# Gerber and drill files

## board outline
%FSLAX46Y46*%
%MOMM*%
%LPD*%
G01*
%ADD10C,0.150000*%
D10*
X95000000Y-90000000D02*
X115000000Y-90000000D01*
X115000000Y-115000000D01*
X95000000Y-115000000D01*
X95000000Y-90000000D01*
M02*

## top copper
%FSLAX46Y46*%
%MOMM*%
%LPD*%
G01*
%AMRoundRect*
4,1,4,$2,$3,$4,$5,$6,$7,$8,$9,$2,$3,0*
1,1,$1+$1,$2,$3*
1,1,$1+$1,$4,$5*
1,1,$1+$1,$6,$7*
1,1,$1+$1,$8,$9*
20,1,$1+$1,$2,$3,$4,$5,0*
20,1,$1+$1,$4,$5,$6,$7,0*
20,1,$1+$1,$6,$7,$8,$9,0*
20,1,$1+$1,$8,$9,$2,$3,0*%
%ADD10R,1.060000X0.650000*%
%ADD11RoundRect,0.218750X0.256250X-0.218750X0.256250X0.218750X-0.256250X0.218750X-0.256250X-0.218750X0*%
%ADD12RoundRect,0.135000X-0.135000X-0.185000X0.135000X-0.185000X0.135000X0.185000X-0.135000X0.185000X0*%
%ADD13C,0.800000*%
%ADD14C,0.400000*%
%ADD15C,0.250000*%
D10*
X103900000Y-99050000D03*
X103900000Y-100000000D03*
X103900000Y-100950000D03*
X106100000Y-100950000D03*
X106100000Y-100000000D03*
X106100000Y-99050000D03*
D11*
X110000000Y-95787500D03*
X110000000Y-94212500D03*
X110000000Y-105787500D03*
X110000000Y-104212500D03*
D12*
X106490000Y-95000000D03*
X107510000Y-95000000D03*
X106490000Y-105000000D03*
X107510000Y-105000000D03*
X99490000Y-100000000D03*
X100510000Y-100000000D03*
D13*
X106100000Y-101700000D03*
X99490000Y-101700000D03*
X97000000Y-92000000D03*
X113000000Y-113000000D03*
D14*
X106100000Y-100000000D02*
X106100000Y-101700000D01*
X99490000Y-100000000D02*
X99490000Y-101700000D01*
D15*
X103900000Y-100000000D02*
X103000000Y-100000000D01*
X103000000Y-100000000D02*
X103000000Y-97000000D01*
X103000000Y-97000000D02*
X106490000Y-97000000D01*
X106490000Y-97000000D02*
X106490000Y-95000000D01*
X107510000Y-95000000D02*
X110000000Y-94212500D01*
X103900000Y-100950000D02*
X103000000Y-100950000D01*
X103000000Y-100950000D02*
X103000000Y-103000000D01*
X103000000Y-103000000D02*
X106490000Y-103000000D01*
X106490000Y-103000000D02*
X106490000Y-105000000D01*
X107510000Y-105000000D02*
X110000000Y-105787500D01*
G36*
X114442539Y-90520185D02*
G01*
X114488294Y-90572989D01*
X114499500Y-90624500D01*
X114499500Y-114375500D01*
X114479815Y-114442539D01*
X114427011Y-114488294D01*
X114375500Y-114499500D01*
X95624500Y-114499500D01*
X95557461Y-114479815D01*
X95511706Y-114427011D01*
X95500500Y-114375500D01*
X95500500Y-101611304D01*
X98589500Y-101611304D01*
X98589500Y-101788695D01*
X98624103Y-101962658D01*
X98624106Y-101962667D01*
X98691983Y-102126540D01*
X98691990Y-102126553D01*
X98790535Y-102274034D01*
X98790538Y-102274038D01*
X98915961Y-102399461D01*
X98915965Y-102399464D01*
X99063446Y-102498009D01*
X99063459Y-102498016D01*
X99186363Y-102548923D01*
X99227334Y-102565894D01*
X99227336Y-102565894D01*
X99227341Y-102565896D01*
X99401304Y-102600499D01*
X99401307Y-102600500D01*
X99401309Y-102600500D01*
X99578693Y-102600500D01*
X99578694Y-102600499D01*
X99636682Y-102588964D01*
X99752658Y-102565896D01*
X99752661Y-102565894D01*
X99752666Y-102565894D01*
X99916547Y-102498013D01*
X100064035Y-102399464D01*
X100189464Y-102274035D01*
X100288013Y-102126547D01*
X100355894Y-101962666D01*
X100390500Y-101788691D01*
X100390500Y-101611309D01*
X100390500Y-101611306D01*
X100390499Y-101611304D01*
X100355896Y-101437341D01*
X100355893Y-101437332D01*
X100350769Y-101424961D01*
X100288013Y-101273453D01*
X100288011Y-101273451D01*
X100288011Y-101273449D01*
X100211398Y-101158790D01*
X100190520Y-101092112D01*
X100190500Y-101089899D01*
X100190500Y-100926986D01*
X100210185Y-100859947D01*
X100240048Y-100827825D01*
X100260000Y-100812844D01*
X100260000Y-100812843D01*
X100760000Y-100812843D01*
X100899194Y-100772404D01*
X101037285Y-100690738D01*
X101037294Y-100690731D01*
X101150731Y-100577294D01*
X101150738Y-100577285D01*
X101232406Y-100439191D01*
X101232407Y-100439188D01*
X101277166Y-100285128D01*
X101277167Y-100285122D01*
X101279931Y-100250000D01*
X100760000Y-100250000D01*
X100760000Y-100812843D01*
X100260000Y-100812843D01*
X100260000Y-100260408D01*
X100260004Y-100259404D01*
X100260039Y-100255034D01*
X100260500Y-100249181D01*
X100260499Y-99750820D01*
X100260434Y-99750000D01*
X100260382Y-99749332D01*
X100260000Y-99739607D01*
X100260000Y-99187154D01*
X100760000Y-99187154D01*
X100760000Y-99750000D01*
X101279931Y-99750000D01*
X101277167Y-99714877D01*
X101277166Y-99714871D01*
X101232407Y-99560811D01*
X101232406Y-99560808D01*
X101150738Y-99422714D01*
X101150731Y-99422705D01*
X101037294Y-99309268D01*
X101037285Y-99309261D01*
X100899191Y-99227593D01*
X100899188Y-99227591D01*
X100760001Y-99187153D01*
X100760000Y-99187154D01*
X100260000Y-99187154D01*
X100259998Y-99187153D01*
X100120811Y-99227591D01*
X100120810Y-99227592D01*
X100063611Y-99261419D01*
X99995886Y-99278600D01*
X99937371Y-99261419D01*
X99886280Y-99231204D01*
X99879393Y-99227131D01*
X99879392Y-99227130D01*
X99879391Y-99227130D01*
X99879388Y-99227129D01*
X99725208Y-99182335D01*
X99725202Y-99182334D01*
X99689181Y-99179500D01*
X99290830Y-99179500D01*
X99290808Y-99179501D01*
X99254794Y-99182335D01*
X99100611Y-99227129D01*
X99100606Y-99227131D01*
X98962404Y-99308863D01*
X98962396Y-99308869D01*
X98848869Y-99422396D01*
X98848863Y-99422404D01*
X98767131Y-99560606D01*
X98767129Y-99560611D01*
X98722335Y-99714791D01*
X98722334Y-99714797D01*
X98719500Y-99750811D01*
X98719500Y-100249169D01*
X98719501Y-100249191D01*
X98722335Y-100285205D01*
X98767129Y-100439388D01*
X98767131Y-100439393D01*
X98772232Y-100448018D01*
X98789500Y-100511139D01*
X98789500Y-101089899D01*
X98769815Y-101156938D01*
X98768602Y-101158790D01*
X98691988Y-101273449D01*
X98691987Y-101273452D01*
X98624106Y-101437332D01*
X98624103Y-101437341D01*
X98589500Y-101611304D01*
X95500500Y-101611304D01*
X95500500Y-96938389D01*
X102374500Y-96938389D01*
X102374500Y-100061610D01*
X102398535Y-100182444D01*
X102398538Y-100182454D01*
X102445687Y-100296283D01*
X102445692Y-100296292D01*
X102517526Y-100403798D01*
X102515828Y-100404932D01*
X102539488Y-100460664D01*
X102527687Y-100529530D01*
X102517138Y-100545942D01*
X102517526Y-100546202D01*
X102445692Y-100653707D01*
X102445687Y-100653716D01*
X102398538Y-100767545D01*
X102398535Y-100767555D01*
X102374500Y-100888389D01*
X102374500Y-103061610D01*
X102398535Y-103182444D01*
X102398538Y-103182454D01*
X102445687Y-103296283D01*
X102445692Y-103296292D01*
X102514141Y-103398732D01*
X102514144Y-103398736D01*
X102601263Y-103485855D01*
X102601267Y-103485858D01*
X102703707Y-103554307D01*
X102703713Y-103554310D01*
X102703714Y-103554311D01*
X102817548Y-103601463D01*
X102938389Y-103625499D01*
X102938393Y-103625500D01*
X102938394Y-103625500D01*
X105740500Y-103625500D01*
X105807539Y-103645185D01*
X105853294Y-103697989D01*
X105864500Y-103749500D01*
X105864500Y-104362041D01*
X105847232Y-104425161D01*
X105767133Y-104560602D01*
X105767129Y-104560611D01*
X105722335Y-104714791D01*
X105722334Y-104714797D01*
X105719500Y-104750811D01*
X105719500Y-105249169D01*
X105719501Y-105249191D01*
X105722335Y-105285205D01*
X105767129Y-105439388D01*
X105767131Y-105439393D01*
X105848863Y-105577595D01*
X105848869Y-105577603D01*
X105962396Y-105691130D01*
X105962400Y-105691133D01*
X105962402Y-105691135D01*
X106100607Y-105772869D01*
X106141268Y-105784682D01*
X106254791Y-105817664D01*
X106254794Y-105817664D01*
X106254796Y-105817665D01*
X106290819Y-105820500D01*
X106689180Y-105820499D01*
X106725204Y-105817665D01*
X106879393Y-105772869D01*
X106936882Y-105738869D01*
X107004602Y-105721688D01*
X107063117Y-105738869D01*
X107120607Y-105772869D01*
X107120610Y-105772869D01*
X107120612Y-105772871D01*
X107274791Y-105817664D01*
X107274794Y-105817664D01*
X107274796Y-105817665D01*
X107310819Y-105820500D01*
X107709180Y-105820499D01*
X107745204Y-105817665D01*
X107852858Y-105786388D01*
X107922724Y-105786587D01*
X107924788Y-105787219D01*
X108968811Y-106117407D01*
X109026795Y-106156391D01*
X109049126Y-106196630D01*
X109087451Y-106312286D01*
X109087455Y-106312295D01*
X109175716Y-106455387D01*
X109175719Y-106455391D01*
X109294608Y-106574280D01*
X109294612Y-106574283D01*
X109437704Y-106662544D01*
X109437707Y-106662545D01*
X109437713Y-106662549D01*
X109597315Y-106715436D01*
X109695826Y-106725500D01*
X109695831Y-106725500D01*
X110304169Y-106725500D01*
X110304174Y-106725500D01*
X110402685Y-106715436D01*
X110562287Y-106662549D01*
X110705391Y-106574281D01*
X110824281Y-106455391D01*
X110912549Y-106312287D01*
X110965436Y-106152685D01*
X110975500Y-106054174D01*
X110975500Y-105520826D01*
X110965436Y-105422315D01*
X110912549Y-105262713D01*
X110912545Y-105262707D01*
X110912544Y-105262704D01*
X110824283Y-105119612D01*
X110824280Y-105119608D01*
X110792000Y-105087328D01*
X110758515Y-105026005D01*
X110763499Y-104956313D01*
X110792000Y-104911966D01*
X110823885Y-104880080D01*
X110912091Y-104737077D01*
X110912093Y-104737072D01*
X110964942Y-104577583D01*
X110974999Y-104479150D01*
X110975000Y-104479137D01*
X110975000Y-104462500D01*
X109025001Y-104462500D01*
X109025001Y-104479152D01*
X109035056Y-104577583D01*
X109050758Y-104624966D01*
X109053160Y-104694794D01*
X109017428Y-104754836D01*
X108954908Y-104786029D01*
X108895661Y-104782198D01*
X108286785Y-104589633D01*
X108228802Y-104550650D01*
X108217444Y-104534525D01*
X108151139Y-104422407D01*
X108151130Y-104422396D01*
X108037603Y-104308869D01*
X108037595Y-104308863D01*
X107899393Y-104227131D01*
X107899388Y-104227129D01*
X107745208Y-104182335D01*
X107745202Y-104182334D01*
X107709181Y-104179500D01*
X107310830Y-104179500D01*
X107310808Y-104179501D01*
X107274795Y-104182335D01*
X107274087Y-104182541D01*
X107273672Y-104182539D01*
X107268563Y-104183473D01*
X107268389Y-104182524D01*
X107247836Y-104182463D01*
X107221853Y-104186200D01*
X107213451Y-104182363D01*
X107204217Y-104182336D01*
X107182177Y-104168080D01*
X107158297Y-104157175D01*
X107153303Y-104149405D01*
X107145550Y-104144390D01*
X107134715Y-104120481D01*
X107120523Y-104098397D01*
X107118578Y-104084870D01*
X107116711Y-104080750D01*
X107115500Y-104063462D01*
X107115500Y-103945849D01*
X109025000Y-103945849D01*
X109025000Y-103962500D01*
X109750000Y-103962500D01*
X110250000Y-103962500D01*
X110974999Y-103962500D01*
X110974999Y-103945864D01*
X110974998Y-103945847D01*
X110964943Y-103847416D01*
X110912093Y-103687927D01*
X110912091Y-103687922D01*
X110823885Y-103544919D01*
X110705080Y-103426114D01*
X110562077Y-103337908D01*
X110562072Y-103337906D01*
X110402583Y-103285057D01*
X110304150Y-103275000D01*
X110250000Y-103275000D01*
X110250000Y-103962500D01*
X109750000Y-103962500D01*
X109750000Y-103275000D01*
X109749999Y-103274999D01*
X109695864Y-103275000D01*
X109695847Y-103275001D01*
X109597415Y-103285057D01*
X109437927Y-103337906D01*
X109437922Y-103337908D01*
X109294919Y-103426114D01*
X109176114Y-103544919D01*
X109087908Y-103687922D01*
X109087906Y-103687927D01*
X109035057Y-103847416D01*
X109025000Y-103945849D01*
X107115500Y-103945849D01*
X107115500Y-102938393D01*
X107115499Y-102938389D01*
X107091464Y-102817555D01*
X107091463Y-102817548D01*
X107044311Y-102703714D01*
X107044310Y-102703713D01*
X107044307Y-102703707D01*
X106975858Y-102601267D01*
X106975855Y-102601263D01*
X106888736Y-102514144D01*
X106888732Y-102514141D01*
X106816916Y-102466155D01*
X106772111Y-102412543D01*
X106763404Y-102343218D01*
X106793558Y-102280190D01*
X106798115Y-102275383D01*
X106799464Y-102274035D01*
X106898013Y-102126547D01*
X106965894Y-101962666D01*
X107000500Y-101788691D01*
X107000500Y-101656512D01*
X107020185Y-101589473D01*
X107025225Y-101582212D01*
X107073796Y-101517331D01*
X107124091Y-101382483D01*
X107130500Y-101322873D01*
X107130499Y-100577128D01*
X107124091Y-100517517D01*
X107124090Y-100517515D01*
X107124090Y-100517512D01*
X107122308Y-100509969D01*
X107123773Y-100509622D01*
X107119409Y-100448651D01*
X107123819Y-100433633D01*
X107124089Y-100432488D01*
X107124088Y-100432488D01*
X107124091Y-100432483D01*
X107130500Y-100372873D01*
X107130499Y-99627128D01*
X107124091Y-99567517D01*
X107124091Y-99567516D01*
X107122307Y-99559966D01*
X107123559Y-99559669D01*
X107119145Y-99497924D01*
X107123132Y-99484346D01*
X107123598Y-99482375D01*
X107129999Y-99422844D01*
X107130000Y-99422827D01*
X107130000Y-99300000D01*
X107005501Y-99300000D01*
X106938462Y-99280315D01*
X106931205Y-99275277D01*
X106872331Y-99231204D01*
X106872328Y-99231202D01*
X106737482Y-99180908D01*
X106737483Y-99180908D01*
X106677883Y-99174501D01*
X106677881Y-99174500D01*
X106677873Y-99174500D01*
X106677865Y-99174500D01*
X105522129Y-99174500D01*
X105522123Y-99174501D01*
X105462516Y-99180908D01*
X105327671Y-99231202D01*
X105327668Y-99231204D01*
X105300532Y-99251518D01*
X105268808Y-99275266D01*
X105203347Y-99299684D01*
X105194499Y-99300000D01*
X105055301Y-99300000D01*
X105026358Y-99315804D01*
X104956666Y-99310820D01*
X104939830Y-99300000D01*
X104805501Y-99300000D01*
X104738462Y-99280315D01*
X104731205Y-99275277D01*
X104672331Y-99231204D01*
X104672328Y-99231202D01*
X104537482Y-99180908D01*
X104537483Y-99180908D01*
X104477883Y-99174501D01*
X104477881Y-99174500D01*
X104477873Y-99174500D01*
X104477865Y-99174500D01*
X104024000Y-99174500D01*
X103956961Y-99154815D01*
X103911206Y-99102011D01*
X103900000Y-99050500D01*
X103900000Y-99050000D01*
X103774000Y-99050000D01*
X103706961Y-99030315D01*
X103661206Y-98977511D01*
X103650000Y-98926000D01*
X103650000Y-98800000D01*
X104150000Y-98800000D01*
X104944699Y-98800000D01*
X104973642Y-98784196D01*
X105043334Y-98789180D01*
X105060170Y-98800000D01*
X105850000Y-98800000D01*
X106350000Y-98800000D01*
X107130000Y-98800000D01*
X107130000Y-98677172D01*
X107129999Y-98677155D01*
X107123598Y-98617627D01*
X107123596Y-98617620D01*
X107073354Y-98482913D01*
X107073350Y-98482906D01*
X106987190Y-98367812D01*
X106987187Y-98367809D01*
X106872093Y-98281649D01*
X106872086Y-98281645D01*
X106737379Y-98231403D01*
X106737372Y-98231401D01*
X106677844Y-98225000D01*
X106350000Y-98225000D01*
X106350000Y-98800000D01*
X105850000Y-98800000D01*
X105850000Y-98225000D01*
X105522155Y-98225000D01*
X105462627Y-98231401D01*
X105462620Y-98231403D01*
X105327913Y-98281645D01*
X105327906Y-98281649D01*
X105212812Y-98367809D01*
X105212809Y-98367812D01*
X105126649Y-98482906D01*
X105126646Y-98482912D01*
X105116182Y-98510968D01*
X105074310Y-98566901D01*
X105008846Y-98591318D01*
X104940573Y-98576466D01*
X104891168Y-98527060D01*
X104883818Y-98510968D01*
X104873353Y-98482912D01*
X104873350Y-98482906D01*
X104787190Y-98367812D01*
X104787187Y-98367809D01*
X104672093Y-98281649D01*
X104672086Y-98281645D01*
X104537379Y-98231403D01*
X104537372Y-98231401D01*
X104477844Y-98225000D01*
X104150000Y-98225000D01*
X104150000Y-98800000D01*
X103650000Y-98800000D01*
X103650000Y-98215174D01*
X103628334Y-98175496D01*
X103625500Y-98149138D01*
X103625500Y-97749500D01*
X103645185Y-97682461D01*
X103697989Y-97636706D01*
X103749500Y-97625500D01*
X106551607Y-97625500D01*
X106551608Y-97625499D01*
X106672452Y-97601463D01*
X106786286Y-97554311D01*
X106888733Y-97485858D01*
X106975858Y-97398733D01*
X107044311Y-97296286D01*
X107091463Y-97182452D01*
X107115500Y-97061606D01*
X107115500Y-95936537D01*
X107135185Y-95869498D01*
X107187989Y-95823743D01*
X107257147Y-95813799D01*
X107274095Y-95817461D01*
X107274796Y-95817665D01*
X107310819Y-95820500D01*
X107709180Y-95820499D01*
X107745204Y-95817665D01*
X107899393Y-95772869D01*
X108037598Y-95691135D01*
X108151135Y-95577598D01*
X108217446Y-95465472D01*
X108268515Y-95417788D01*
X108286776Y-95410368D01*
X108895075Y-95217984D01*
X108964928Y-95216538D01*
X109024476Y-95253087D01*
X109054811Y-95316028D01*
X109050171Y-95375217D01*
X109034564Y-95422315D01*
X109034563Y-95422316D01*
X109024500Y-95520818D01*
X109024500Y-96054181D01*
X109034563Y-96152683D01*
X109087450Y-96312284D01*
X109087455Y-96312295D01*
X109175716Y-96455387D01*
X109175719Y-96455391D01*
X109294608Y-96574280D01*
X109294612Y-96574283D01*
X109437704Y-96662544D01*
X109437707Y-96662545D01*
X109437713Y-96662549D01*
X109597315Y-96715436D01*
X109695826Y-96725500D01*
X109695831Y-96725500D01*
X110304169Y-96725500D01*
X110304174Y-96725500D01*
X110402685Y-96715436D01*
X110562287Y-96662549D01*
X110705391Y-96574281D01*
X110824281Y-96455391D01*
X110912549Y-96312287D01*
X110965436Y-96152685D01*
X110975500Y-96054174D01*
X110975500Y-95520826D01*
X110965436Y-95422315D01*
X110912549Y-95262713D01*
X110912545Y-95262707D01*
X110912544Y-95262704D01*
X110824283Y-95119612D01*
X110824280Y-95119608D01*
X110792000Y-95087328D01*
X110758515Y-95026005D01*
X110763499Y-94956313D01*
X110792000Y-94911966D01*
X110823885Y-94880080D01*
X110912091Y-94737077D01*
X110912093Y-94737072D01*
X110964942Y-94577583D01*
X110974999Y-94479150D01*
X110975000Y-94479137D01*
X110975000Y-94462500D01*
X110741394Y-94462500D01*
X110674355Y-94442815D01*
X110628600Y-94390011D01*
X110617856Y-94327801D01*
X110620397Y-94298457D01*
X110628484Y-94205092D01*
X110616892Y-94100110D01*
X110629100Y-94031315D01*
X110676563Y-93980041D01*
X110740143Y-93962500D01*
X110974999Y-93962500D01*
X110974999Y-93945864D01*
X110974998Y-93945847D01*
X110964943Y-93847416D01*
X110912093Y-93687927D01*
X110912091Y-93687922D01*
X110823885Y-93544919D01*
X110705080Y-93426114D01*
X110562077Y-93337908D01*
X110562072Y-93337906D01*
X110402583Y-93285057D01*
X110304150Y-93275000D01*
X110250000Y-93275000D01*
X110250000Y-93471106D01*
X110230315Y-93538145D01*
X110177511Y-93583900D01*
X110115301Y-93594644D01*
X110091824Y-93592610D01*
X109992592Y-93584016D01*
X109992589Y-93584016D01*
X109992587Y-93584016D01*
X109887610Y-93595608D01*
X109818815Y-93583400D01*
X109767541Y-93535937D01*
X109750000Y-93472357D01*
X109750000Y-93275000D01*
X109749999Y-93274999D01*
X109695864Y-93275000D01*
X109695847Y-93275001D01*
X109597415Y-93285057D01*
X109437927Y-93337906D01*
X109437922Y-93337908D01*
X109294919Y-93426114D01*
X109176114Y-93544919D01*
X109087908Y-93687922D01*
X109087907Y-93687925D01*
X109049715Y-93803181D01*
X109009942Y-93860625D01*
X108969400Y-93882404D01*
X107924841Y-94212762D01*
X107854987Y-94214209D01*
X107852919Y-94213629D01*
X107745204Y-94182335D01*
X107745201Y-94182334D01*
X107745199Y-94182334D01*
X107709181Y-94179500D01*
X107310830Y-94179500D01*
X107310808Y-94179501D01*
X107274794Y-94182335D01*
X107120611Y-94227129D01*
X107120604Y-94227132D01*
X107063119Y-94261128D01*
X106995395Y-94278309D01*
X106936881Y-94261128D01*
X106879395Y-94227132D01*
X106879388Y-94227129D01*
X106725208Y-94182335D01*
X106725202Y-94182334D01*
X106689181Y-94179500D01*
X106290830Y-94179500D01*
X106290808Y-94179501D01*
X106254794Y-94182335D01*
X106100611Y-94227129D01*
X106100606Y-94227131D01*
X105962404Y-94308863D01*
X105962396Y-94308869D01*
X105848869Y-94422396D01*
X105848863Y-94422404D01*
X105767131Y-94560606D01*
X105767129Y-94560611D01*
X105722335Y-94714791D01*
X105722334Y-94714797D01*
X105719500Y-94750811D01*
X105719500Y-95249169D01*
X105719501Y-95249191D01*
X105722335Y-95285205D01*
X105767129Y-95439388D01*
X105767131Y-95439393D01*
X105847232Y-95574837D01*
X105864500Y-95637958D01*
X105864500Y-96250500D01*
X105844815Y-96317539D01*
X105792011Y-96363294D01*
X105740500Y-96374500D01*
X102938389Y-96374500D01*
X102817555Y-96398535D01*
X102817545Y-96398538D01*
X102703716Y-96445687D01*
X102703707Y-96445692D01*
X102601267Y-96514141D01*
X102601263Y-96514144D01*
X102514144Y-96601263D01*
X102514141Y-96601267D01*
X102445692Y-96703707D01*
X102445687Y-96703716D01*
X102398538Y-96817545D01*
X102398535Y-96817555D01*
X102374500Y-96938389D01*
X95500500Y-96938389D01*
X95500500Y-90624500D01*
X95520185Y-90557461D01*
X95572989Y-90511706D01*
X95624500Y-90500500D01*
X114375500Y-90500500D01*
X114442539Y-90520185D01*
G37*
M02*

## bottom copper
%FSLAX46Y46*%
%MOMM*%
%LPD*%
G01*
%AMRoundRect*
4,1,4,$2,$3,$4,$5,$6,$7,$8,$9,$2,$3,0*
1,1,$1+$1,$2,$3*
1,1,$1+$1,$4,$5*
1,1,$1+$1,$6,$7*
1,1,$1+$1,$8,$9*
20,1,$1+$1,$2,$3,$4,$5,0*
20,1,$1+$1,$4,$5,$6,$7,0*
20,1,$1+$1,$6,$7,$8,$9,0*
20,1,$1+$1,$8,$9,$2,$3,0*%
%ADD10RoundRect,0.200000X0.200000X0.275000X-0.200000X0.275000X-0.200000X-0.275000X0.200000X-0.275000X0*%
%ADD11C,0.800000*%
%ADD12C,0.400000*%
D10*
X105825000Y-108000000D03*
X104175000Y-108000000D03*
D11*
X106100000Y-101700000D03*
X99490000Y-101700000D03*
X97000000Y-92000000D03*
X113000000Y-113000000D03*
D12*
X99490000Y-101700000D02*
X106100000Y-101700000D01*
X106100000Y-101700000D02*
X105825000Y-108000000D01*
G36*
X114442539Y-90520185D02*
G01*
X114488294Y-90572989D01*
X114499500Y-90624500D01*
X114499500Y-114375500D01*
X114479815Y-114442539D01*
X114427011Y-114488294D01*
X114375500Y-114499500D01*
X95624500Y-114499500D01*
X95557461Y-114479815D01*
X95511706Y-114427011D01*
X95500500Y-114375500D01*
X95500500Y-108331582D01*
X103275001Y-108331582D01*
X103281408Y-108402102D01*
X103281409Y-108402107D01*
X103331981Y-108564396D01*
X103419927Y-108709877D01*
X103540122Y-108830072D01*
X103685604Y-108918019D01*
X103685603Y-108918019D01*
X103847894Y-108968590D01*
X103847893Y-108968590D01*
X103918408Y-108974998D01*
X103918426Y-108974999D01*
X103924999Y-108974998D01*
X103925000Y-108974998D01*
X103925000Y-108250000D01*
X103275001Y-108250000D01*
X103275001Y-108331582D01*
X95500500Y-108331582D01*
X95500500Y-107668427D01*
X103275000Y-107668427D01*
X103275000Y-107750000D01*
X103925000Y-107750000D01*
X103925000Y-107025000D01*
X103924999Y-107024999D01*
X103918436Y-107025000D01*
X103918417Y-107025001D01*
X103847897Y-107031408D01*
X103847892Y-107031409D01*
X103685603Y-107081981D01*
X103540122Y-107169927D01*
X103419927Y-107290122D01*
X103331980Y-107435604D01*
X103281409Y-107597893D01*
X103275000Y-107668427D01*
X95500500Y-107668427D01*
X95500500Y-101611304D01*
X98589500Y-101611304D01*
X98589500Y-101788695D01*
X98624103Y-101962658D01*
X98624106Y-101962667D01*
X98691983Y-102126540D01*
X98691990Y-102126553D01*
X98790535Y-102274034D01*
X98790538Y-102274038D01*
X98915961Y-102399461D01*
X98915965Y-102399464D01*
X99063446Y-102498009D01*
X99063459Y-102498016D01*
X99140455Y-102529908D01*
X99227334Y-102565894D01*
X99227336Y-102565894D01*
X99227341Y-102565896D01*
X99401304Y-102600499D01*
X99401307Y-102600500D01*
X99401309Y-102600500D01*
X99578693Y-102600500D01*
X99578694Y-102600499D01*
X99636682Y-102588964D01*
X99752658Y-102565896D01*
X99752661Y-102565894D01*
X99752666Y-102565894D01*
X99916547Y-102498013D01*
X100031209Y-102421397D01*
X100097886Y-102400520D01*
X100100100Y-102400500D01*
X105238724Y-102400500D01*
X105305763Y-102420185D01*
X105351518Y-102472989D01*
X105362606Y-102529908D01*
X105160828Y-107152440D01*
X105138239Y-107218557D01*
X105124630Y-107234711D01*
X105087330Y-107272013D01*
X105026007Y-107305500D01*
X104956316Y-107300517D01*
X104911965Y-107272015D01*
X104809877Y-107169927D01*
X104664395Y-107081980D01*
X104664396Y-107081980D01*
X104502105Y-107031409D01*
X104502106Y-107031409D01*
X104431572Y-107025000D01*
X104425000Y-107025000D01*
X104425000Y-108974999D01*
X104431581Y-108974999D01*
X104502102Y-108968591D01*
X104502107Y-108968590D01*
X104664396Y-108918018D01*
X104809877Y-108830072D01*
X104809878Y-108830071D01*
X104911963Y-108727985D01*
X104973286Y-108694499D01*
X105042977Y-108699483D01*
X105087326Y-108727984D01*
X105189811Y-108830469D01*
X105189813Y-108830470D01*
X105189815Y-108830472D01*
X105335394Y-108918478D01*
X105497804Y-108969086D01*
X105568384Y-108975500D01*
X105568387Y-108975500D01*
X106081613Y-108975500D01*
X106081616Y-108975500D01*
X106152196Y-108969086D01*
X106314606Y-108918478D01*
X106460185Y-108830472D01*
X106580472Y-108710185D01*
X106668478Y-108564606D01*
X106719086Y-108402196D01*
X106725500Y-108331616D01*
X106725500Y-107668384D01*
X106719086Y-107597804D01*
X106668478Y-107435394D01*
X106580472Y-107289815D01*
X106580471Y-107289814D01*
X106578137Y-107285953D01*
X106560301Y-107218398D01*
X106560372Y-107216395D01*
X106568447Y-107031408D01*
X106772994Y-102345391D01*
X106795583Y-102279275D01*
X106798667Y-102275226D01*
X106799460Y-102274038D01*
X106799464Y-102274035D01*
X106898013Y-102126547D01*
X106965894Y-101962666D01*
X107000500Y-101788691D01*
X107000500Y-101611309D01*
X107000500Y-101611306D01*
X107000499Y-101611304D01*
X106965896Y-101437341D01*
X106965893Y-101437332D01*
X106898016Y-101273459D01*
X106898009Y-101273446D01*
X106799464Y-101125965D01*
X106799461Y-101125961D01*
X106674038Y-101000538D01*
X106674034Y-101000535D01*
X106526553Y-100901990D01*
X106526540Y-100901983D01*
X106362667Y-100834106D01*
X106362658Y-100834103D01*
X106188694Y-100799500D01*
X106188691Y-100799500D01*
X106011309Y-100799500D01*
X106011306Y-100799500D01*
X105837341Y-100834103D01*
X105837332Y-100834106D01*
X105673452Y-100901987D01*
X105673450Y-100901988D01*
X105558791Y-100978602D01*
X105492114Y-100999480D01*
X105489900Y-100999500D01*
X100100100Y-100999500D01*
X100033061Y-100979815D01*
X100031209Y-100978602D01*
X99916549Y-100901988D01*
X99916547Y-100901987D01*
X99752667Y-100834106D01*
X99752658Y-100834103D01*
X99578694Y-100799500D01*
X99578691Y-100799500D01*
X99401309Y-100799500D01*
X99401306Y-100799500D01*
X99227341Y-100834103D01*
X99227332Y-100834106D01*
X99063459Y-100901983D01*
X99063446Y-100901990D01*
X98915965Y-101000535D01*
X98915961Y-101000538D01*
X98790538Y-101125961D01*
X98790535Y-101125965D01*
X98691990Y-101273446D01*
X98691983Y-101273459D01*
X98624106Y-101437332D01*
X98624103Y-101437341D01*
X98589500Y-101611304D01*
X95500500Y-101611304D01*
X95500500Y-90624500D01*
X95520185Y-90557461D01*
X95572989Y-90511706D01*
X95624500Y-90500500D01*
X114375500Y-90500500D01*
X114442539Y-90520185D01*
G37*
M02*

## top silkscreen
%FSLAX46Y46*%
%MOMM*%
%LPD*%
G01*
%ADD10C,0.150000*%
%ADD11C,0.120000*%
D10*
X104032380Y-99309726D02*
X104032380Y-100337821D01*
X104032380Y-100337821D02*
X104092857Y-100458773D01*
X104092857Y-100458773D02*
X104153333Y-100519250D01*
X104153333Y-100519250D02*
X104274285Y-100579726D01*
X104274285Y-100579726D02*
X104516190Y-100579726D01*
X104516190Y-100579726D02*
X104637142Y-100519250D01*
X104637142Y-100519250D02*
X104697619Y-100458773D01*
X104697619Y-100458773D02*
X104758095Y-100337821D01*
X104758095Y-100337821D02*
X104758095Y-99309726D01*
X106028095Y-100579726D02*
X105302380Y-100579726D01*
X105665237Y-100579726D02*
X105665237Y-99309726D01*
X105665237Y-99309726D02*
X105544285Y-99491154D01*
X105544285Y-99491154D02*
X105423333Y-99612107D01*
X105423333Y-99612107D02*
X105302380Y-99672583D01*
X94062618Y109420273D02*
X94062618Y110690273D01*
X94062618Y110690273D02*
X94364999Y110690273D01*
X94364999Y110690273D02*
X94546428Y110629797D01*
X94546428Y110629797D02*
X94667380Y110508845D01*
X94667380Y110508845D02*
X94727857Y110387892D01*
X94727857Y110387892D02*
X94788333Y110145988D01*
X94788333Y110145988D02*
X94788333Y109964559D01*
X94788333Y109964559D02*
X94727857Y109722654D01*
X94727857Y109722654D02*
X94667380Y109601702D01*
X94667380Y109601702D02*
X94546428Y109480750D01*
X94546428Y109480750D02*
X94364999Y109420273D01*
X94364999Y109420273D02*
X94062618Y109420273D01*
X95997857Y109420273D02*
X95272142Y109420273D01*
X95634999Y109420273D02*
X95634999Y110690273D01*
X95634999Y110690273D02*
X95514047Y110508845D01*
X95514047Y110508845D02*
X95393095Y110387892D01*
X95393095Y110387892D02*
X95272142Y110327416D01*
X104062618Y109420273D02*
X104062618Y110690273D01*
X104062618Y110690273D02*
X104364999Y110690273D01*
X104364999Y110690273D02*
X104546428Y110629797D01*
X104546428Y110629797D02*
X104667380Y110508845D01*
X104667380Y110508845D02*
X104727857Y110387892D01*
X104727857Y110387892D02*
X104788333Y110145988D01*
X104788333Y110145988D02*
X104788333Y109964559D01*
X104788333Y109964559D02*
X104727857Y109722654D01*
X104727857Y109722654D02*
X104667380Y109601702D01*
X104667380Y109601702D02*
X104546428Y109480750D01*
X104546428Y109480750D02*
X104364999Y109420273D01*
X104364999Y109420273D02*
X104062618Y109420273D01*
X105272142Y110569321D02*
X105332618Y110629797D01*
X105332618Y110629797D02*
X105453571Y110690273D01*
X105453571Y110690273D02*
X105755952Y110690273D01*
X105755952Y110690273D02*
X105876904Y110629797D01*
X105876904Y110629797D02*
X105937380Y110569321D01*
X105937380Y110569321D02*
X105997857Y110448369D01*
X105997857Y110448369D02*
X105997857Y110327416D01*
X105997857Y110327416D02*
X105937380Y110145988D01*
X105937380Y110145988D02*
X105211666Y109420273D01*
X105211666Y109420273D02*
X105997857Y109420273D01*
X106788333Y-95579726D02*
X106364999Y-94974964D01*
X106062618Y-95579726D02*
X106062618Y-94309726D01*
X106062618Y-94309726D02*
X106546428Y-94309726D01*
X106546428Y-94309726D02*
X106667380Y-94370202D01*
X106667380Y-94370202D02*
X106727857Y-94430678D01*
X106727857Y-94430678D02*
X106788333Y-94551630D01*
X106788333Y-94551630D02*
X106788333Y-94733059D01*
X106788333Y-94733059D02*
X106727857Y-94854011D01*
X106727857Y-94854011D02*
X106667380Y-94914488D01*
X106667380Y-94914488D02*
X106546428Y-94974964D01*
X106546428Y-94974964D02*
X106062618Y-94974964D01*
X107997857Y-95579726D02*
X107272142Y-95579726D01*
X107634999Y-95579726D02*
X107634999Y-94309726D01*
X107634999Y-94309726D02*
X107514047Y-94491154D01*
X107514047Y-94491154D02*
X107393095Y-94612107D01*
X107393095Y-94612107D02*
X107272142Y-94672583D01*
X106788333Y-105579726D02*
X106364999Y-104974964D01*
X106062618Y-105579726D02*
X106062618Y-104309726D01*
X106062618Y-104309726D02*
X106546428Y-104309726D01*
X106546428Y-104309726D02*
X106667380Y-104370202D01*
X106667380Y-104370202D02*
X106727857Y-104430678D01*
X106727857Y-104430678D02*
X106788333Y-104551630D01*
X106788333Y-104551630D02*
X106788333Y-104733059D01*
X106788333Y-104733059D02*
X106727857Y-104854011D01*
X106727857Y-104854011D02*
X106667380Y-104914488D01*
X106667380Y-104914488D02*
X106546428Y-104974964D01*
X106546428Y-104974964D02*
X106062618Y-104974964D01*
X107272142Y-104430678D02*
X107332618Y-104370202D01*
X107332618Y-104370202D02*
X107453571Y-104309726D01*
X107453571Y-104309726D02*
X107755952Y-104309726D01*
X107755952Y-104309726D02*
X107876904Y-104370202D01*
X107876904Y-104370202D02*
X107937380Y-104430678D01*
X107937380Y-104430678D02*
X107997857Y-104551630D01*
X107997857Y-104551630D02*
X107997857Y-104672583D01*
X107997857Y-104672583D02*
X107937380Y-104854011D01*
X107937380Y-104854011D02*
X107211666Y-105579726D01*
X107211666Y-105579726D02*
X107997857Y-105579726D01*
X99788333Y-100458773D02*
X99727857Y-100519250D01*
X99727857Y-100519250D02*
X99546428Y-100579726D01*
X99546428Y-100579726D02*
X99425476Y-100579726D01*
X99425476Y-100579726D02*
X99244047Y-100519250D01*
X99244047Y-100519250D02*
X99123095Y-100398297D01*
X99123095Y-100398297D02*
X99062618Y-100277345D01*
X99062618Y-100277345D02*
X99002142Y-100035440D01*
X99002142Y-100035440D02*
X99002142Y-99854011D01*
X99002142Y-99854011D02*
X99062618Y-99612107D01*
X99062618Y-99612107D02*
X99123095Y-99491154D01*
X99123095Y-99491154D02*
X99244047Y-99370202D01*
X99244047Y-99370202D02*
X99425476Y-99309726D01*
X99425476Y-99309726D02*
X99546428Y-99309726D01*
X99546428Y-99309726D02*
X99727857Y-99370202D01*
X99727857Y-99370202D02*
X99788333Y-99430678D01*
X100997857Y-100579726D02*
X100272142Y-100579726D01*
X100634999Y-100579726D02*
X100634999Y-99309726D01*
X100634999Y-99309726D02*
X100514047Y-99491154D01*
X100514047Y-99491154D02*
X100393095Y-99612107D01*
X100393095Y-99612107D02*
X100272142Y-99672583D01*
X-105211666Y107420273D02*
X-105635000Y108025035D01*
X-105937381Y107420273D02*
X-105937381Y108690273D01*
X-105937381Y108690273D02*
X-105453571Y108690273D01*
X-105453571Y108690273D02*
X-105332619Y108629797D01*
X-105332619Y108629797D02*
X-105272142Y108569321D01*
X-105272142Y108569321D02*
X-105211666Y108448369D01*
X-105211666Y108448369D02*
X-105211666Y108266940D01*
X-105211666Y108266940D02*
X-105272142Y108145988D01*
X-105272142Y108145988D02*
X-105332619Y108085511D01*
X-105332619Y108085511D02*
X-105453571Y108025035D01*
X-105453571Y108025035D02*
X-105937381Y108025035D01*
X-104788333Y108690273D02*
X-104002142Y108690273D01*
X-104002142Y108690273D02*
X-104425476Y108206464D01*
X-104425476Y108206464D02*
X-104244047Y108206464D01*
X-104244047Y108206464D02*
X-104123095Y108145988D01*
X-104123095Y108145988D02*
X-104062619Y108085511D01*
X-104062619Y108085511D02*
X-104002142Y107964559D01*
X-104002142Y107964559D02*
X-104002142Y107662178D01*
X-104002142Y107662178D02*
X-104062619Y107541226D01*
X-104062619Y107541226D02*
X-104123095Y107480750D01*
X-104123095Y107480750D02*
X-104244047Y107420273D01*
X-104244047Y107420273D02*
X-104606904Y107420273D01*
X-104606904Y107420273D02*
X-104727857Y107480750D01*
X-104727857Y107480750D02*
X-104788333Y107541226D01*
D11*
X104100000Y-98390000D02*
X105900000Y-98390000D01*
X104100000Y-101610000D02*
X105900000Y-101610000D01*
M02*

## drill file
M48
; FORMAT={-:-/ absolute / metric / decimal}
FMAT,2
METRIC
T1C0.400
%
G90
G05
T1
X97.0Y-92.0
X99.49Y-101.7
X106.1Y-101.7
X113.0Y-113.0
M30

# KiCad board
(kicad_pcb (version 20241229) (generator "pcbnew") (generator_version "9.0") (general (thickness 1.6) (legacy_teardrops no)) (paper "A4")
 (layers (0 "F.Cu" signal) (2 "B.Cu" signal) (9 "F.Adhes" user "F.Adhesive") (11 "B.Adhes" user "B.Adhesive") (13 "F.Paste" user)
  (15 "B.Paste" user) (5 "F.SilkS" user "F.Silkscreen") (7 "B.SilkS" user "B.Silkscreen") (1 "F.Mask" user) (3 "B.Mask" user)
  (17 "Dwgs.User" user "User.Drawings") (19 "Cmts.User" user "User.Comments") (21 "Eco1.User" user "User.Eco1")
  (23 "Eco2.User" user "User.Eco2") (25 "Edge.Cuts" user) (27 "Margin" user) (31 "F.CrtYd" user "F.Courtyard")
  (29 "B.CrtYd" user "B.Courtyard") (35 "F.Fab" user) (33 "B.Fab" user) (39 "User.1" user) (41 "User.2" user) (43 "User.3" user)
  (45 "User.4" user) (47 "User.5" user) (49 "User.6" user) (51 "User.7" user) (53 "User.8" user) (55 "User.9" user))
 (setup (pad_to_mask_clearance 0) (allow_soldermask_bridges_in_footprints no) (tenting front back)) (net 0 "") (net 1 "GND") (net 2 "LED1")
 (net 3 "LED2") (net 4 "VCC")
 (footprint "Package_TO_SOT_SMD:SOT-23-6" (layer "F.Cu") (at 105 100)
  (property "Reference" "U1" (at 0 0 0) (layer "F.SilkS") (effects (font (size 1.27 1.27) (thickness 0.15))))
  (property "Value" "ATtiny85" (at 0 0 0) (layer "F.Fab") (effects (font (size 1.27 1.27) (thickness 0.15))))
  (fp_line (start -0.9 -1.61) (end 0.9 -1.61) (stroke (width 0.12) (type solid)) (layer "F.SilkS"))
  (fp_line (start -0.9 1.61) (end 0.9 1.61) (stroke (width 0.12) (type solid)) (layer "F.SilkS"))
  (pad "1" smd rect (at -1.1 -0.95) (size 1.06 0.65) (layers "F.Cu" "F.Mask" "F.Paste") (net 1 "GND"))
  (pad "2" smd rect (at -1.1 0) (size 1.06 0.65) (layers "F.Cu" "F.Mask" "F.Paste") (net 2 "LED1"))
  (pad "3" smd rect (at -1.1 0.95) (size 1.06 0.65) (layers "F.Cu" "F.Mask" "F.Paste") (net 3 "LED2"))
  (pad "4" smd rect (at 1.1 0.95) (size 1.06 0.65) (layers "F.Cu" "F.Mask" "F.Paste") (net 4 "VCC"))
  (pad "5" smd rect (at 1.1 0) (size 1.06 0.65) (layers "F.Cu" "F.Mask" "F.Paste") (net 4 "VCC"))
  (pad "6" smd rect (at 1.1 -0.95) (size 1.06 0.65) (layers "F.Cu" "F.Mask" "F.Paste") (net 1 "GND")))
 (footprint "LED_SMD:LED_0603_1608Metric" (layer "F.Cu") (at 110 95 90)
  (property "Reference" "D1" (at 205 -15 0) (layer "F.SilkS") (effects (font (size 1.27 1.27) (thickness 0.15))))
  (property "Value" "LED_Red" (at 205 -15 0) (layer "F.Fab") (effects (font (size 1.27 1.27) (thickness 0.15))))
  (pad "1" smd roundrect (at -0.7875 0 90) (size 0.875 0.95) (layers "F.Cu" "F.Mask" "F.Paste") (roundrect_rratio 0.25) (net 2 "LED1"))
  (pad "2" smd roundrect (at 0.7875 0 90) (size 0.875 0.95) (layers "F.Cu" "F.Mask" "F.Paste") (roundrect_rratio 0.25) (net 1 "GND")))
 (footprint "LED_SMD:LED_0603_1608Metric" (layer "F.Cu") (at 110 105 90)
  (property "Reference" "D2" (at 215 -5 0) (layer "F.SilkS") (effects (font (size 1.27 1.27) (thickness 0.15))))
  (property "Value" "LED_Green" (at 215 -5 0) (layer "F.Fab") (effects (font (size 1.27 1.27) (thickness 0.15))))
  (pad "1" smd roundrect (at -0.7875 0 90) (size 0.875 0.95) (layers "F.Cu" "F.Mask" "F.Paste") (roundrect_rratio 0.25) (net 3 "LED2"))
  (pad "2" smd roundrect (at 0.7875 0 90) (size 0.875 0.95) (layers "F.Cu" "F.Mask" "F.Paste") (roundrect_rratio 0.25) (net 1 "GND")))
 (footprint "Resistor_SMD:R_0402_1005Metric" (layer "F.Cu") (at 107 95)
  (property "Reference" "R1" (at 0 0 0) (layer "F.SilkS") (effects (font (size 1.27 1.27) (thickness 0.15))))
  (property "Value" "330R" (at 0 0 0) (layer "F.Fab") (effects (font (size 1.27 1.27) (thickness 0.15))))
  (pad "1" smd roundrect (at -0.51 0) (size 0.54 0.64) (layers "F.Cu" "F.Mask" "F.Paste") (roundrect_rratio 0.25) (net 2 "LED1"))
  (pad "2" smd roundrect (at 0.51 0) (size 0.54 0.64) (layers "F.Cu" "F.Mask" "F.Paste") (roundrect_rratio 0.25) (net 2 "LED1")))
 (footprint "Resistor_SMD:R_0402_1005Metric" (layer "F.Cu") (at 107 105)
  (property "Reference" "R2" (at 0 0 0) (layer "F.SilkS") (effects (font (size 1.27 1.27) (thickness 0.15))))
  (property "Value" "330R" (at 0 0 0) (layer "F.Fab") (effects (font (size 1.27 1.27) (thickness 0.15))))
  (pad "1" smd roundrect (at -0.51 0) (size 0.54 0.64) (layers "F.Cu" "F.Mask" "F.Paste") (roundrect_rratio 0.25) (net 3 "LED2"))
  (pad "2" smd roundrect (at 0.51 0) (size 0.54 0.64) (layers "F.Cu" "F.Mask" "F.Paste") (roundrect_rratio 0.25) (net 3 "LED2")))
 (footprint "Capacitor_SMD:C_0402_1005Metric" (layer "F.Cu") (at 100 100)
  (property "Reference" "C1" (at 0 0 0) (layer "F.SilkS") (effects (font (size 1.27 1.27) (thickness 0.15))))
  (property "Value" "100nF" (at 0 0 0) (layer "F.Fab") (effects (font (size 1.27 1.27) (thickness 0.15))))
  (pad "1" smd roundrect (at -0.51 0) (size 0.54 0.64) (layers "F.Cu" "F.Mask" "F.Paste") (roundrect_rratio 0.25) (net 4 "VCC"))
  (pad "2" smd roundrect (at 0.51 0) (size 0.54 0.64) (layers "F.Cu" "F.Mask" "F.Paste") (roundrect_rratio 0.25) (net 1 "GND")))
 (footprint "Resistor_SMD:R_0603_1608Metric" (layer "B.Cu") (at 105 108 180)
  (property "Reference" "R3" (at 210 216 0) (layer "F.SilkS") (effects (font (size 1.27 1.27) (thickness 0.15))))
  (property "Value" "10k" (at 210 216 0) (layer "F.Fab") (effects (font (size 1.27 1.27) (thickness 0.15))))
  (pad "1" smd roundrect (at -0.825 0 180) (size 0.8 0.95) (layers "B.Cu" "B.Mask" "B.Paste") (roundrect_rratio 0.25) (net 4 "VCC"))
  (pad "2" smd roundrect (at 0.825 0 180) (size 0.8 0.95) (layers "B.Cu" "B.Mask" "B.Paste") (roundrect_rratio 0.25) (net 1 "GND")))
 (gr_rect (start 95 90) (end 115 115) (stroke (width 0.15) (type solid)) (fill no) (layer "Edge.Cuts"))
 (segment (start 106.1 100) (end 106.1 101.7) (width 0.4) (layer "F.Cu") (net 4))
 (segment (start 99.49 100) (end 99.49 101.7) (width 0.4) (layer "F.Cu") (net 4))
 (via (at 106.1 101.7) (size 0.8) (drill 0.4) (layers "F.Cu" "B.Cu") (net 4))
 (via (at 99.49 101.7) (size 0.8) (drill 0.4) (layers "F.Cu" "B.Cu") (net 4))
 (segment (start 99.49 101.7) (end 106.1 101.7) (width 0.4) (layer "B.Cu") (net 4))
 (segment (start 106.1 101.7) (end 105.825 108) (width 0.4) (layer "B.Cu") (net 4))
 (via (at 97 92) (size 0.8) (drill 0.4) (layers "F.Cu" "B.Cu") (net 1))
 (via (at 113 113) (size 0.8) (drill 0.4) (layers "F.Cu" "B.Cu") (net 1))
 (segment (start 103.9 100) (end 103 100) (width 0.25) (layer "F.Cu") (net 2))
 (segment (start 103 100) (end 103 97) (width 0.25) (layer "F.Cu") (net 2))
 (segment (start 103 97) (end 106.49 97) (width 0.25) (layer "F.Cu") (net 2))
 (segment (start 106.49 97) (end 106.49 95) (width 0.25) (layer "F.Cu") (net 2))
 (segment (start 107.51 95) (end 110 94.2125) (width 0.25) (layer "F.Cu") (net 2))
 (segment (start 103.9 100.95) (end 103 100.95) (width 0.25) (layer "F.Cu") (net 3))
 (segment (start 103 100.95) (end 103 103) (width 0.25) (layer "F.Cu") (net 3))
 (segment (start 103 103) (end 106.49 103) (width 0.25) (layer "F.Cu") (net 3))
 (segment (start 106.49 103) (end 106.49 105) (width 0.25) (layer "F.Cu") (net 3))
 (segment (start 107.51 105) (end 110 105.7875) (width 0.25) (layer "F.Cu") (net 3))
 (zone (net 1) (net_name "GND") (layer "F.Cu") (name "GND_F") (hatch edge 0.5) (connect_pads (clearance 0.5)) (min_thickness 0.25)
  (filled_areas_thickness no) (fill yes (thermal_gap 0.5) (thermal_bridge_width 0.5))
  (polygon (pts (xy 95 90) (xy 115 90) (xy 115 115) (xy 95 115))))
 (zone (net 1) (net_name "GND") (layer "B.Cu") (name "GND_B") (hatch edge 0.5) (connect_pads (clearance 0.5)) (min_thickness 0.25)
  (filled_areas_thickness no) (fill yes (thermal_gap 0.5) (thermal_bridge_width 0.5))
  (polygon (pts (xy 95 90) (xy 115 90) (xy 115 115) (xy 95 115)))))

